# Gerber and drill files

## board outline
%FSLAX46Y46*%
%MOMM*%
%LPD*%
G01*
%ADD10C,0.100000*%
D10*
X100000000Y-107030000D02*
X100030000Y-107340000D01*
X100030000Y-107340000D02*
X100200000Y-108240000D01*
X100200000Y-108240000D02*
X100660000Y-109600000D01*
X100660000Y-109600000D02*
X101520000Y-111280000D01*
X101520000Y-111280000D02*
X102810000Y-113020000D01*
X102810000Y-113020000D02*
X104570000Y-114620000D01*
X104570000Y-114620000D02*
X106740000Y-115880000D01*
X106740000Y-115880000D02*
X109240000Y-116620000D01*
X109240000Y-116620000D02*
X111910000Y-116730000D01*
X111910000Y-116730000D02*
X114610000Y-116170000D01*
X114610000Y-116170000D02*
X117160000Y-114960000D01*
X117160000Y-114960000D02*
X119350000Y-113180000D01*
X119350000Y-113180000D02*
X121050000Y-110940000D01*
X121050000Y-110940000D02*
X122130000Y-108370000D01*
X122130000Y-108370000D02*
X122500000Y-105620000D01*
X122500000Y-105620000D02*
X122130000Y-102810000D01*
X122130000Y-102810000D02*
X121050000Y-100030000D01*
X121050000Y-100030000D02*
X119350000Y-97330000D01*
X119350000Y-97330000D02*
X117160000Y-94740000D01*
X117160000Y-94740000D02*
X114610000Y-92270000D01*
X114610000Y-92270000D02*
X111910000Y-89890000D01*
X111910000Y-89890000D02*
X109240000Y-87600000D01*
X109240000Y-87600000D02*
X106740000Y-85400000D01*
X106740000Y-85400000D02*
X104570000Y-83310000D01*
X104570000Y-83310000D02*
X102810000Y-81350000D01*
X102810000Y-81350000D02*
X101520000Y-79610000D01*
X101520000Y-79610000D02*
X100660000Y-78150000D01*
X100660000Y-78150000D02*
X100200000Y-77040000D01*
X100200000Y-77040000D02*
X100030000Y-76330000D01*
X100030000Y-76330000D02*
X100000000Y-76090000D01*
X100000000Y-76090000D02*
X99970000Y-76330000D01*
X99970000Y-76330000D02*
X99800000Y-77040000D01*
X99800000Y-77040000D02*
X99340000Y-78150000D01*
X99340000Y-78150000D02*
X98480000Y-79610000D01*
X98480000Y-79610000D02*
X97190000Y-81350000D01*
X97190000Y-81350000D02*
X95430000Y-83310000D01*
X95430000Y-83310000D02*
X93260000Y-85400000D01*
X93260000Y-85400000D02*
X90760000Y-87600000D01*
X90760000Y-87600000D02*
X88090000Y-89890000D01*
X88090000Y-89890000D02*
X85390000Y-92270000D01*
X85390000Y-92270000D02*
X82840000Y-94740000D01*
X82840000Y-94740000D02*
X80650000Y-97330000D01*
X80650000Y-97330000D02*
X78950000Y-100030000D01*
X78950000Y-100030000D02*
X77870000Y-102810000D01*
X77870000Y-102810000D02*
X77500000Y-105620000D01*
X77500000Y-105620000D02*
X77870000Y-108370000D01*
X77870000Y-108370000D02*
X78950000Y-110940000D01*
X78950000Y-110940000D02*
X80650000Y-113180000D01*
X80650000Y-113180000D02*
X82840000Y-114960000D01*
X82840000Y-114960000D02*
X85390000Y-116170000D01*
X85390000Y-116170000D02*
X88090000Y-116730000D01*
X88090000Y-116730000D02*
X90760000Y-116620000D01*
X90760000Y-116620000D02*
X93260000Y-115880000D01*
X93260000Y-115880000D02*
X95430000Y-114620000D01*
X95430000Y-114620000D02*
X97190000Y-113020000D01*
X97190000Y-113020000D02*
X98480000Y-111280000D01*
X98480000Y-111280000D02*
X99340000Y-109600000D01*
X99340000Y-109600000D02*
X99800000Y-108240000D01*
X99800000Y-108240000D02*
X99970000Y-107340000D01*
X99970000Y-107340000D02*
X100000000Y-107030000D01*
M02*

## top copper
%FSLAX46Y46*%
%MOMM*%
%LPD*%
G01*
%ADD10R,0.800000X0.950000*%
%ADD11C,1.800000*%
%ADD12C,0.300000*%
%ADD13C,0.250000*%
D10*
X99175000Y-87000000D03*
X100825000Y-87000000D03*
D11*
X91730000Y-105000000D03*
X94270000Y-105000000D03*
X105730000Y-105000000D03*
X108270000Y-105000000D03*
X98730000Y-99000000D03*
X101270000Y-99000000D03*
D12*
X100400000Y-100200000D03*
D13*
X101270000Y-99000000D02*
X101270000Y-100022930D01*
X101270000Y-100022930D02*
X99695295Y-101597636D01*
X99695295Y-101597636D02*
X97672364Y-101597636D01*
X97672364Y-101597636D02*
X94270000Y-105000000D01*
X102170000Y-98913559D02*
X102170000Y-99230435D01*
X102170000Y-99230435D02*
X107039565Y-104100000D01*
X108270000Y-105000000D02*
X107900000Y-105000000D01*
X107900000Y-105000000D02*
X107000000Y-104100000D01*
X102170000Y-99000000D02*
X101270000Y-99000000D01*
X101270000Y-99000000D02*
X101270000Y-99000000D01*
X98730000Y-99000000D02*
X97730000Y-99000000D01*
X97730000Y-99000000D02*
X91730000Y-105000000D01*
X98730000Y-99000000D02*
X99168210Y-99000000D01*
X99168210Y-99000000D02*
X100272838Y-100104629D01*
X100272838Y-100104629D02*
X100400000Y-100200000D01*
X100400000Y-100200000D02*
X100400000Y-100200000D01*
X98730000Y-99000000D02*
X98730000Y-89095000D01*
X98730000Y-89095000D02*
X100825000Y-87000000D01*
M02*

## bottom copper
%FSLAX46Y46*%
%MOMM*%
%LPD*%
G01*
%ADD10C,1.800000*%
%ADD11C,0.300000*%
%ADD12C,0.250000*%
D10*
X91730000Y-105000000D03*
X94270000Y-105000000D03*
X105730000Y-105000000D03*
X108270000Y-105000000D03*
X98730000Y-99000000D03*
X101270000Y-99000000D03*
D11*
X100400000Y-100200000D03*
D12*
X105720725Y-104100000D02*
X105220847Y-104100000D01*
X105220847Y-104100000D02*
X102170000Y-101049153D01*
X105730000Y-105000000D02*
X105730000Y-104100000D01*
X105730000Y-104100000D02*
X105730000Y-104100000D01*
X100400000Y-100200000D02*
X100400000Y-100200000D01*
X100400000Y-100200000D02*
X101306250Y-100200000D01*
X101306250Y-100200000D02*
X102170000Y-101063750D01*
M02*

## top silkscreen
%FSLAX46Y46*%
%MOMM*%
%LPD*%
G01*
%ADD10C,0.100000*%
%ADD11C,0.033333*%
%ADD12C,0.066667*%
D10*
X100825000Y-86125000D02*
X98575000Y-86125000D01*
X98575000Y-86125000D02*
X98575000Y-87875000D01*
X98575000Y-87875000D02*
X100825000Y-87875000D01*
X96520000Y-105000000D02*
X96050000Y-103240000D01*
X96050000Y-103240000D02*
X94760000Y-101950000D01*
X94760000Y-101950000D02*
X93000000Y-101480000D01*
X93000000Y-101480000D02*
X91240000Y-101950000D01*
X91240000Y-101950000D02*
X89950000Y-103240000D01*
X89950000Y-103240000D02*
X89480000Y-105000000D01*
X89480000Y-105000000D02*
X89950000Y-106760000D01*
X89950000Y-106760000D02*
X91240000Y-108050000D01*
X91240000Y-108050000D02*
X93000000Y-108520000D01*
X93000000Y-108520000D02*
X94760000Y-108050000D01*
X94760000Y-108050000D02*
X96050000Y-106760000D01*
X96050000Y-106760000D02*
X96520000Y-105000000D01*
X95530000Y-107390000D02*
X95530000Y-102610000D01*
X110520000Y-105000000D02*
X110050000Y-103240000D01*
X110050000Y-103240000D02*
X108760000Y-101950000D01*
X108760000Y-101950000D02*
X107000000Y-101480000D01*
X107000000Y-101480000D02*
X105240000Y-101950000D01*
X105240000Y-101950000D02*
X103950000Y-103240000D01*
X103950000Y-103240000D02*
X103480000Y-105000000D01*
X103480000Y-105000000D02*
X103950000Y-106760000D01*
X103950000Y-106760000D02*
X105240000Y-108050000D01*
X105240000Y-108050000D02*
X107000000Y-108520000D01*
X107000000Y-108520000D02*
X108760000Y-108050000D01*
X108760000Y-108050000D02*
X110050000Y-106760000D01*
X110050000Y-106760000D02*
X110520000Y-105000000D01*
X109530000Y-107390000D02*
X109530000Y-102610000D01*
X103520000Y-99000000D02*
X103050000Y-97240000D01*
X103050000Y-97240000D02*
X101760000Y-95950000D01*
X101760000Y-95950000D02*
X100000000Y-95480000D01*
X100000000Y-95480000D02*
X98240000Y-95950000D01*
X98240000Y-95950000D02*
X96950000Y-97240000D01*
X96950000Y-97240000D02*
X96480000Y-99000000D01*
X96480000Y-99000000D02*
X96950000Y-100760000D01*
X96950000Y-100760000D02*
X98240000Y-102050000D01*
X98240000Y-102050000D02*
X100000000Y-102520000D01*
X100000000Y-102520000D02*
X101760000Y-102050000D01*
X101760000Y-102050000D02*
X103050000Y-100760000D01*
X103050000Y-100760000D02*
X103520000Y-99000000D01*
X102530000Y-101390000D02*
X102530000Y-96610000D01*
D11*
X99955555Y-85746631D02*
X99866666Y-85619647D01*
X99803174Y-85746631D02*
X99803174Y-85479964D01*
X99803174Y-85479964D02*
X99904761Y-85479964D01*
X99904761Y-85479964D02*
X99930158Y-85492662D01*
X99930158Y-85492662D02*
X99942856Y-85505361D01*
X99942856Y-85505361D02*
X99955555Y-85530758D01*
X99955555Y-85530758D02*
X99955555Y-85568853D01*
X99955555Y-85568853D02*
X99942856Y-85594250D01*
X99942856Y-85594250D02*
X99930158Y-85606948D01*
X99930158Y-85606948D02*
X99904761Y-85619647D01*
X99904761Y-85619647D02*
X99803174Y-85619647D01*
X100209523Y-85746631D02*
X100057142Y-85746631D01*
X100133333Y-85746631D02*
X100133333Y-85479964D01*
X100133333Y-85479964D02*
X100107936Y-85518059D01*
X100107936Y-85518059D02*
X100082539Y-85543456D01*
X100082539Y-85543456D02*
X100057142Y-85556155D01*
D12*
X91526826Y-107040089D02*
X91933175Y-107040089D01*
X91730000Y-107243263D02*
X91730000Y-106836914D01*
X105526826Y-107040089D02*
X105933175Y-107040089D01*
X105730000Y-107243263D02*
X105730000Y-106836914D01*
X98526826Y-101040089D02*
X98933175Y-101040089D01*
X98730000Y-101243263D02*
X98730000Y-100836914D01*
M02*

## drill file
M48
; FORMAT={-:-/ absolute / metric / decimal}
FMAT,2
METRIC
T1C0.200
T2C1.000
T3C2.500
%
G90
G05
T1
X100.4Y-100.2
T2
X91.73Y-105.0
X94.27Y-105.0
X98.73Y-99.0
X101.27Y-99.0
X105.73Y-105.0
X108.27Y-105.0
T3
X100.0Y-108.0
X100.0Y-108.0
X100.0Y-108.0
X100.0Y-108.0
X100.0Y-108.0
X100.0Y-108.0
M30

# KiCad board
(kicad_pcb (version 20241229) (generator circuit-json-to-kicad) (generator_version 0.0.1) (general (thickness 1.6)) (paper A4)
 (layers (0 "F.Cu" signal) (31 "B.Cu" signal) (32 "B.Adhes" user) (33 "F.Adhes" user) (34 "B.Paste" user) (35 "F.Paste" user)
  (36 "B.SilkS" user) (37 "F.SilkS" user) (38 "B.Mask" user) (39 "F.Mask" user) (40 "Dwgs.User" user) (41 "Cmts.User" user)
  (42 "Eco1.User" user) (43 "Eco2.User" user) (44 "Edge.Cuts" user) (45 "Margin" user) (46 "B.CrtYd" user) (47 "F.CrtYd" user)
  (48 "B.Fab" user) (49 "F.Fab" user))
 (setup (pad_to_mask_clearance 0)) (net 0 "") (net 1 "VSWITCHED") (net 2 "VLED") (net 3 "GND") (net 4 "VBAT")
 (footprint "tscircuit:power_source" (layer F.Cu) (at 100 95 0)
  (pad "" np_thru_hole circle (at 0 13 0) (size 2.5 2.5) (drill 2.5) (layers *.Cu *.Mask)))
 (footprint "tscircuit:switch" (layer F.Cu) (at 100 90 0)
  (pad "" np_thru_hole circle (at 0 18 0) (size 2.5 2.5) (drill 2.5) (layers *.Cu *.Mask)))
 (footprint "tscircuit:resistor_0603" (layer F.Cu) (at 100 87 0)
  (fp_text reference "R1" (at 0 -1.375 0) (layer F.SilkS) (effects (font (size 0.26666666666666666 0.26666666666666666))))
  (pad "1" smd rect (at -0.825 0 0) (size 0.8 0.95) (layers F.Cu F.Paste F.Mask) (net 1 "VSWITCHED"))
  (pad "2" smd rect (at 0.825 0 0) (size 0.8 0.95) (layers F.Cu F.Paste F.Mask) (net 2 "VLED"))
  (pad "" np_thru_hole circle (at 0 21 0) (size 2.5 2.5) (drill 2.5) (layers *.Cu *.Mask)))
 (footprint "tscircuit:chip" (layer F.Cu) (at 93 105 0)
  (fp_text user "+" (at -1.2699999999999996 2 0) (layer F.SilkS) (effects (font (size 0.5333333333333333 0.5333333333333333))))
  (pad "1" thru_hole circle (at -1.2699999999999996 0 0) (size 1.8 1.8) (drill 1) (layers *.Cu *.Mask) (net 2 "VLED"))
  (pad "2" thru_hole circle (at 1.2699999999999996 0 0) (size 1.8 1.8) (drill 1) (layers *.Cu *.Mask) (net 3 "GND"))
  (pad "" np_thru_hole circle (at 7 3 0) (size 2.5 2.5) (drill 2.5) (layers *.Cu *.Mask)))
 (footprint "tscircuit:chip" (layer F.Cu) (at 107 105 0)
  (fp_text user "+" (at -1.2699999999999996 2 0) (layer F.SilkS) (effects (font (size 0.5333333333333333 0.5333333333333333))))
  (pad "1" thru_hole circle (at -1.2699999999999996 0 0) (size 1.8 1.8) (drill 1) (layers *.Cu *.Mask) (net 2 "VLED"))
  (pad "2" thru_hole circle (at 1.2699999999999996 0 0) (size 1.8 1.8) (drill 1) (layers *.Cu *.Mask) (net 3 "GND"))
  (pad "" np_thru_hole circle (at -7 3 0) (size 2.5 2.5) (drill 2.5) (layers *.Cu *.Mask)))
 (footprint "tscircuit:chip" (layer F.Cu) (at 100 99 0)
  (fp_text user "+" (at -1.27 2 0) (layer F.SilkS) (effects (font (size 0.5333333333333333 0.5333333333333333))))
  (pad "1" thru_hole circle (at -1.27 0 0) (size 1.8 1.8) (drill 1) (layers *.Cu *.Mask) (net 2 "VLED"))
  (pad "2" thru_hole circle (at 1.27 0 0) (size 1.8 1.8) (drill 1) (layers *.Cu *.Mask) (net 3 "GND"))
  (pad "" np_thru_hole circle (at 0 9 0) (size 2.5 2.5) (drill 2.5) (layers *.Cu *.Mask)))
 (segment (start 101.27 99) (end 101.27 100.02293031919105) (width 0.25) (layer F.Cu) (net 3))
 (segment (start 101.27 100.02293031919105) (end 99.69529453119956 101.59763578799148) (width 0.25) (layer F.Cu) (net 3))
 (segment (start 99.69529453119956 101.59763578799148) (end 97.67236421200852 101.59763578799148) (width 0.25) (layer F.Cu) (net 3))
 (segment (start 97.67236421200852 101.59763578799148) (end 94.27 105) (width 0.25) (layer F.Cu) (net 3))
 (segment (start 102.17 98.9135593220339) (end 102.17 99.2304347826087) (width 0.25) (layer F.Cu) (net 3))
 (segment (start 102.17 99.2304347826087) (end 107.0395652173913 104.1) (width 0.25) (layer F.Cu) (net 3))
 (segment (start 108.27 105) (end 107.9 105) (width 0.25) (layer F.Cu) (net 3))
 (segment (start 107.9 105) (end 107 104.1) (width 0.25) (layer F.Cu) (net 3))
 (segment (start 102.17 99) (end 101.27 99) (width 0.25) (layer F.Cu) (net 3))
 (segment (start 101.27 99) (end 101.27 99) (width 0.25) (layer F.Cu) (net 3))
 (segment (start 98.73 99) (end 97.73 99) (width 0.25) (layer F.Cu) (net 2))
 (segment (start 97.73 99) (end 91.73 105) (width 0.25) (layer F.Cu) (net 2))
 (segment (start 105.72072463768116 104.1) (end 105.22084745762712 104.1) (width 0.25) (layer B.Cu) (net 2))
 (segment (start 105.22084745762712 104.1) (end 102.17 101.04915254237288) (width 0.25) (layer B.Cu) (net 2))
 (segment (start 105.73 105) (end 105.73 104.1) (width 0.25) (layer B.Cu) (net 2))
 (segment (start 105.73 104.1) (end 105.73 104.1) (width 0.25) (layer B.Cu) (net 2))
 (segment (start 98.73 99) (end 99.1682096086742 99) (width 0.25) (layer F.Cu) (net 2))
 (segment (start 99.1682096086742 99) (end 100.27283843469682 100.10462882602262) (width 0.25) (layer F.Cu) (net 2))
 (segment (start 100.27283843469682 100.10462882602262) (end 100.4 100.2) (width 0.25) (layer F.Cu) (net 2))
 (segment (start 100.4 100.2) (end 100.4 100.2) (width 0.25) (layer F.Cu) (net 2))
 (segment (start 100.4 100.2) (end 100.4 100.2) (width 0.25) (layer B.Cu) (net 2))
 (segment (start 100.4 100.2) (end 101.30625 100.2) (width 0.25) (layer B.Cu) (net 2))
 (segment (start 101.30625 100.2) (end 102.17 101.06375) (width 0.25) (layer B.Cu) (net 2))
 (segment (start 98.73 99) (end 98.73 89.095) (width 0.25) (layer F.Cu) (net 2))
 (segment (start 98.73 89.095) (end 100.825 87) (width 0.25) (layer F.Cu) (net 2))
 (gr_line (start 100.825 86.125) (end 98.575 86.125) (width 0.1) (layer F.SilkS))
 (gr_line (start 98.575 86.125) (end 98.575 87.875) (width 0.1) (layer F.SilkS))
 (gr_line (start 98.575 87.875) (end 100.825 87.875) (width 0.1) (layer F.SilkS))
 (gr_line (start 96.52 105) (end 96.05 103.24) (width 0.1) (layer F.SilkS))
 (gr_line (start 96.05 103.24) (end 94.76 101.95) (width 0.1) (layer F.SilkS))
 (gr_line (start 94.76 101.95) (end 93 101.48) (width 0.1) (layer F.SilkS))
 (gr_line (start 93 101.48) (end 91.24 101.95) (width 0.1) (layer F.SilkS))
 (gr_line (start 91.24 101.95) (end 89.95 103.24) (width 0.1) (layer F.SilkS))
 (gr_line (start 89.95 103.24) (end 89.48 105) (width 0.1) (layer F.SilkS))
 (gr_line (start 89.48 105) (end 89.95 106.76) (width 0.1) (layer F.SilkS))
 (gr_line (start 89.95 106.76) (end 91.24 108.05) (width 0.1) (layer F.SilkS))
 (gr_line (start 91.24 108.05) (end 93 108.52) (width 0.1) (layer F.SilkS))
 (gr_line (start 93 108.52) (end 94.76 108.05) (width 0.1) (layer F.SilkS))
 (gr_line (start 94.76 108.05) (end 96.05 106.76) (width 0.1) (layer F.SilkS))
 (gr_line (start 96.05 106.76) (end 96.52 105) (width 0.1) (layer F.SilkS))
 (gr_line (start 95.53 107.39) (end 95.53 102.61) (width 0.1) (layer F.SilkS))
 (gr_line (start 110.52 105) (end 110.05 103.24) (width 0.1) (layer F.SilkS))
 (gr_line (start 110.05 103.24) (end 108.76 101.95) (width 0.1) (layer F.SilkS))
 (gr_line (start 108.76 101.95) (end 107 101.48) (width 0.1) (layer F.SilkS))
 (gr_line (start 107 101.48) (end 105.24 101.95) (width 0.1) (layer F.SilkS))
 (gr_line (start 105.24 101.95) (end 103.95 103.24) (width 0.1) (layer F.SilkS))
 (gr_line (start 103.95 103.24) (end 103.48 105) (width 0.1) (layer F.SilkS))
 (gr_line (start 103.48 105) (end 103.95 106.76) (width 0.1) (layer F.SilkS))
 (gr_line (start 103.95 106.76) (end 105.24 108.05) (width 0.1) (layer F.SilkS))
 (gr_line (start 105.24 108.05) (end 107 108.52) (width 0.1) (layer F.SilkS))
 (gr_line (start 107 108.52) (end 108.76 108.05) (width 0.1) (layer F.SilkS))
 (gr_line (start 108.76 108.05) (end 110.05 106.76) (width 0.1) (layer F.SilkS))
 (gr_line (start 110.05 106.76) (end 110.52 105) (width 0.1) (layer F.SilkS))
 (gr_line (start 109.53 107.39) (end 109.53 102.61) (width 0.1) (layer F.SilkS))
 (gr_line (start 103.52 99) (end 103.05 97.24) (width 0.1) (layer F.SilkS))
 (gr_line (start 103.05 97.24) (end 101.76 95.95) (width 0.1) (layer F.SilkS))
 (gr_line (start 101.76 95.95) (end 100 95.48) (width 0.1) (layer F.SilkS))
 (gr_line (start 100 95.48) (end 98.24 95.95) (width 0.1) (layer F.SilkS))
 (gr_line (start 98.24 95.95) (end 96.95 97.24) (width 0.1) (layer F.SilkS))
 (gr_line (start 96.95 97.24) (end 96.48 99) (width 0.1) (layer F.SilkS))
 (gr_line (start 96.48 99) (end 96.95 100.76) (width 0.1) (layer F.SilkS))
 (gr_line (start 96.95 100.76) (end 98.24 102.05) (width 0.1) (layer F.SilkS))
 (gr_line (start 98.24 102.05) (end 100 102.52) (width 0.1) (layer F.SilkS))
 (gr_line (start 100 102.52) (end 101.76 102.05) (width 0.1) (layer F.SilkS))
 (gr_line (start 101.76 102.05) (end 103.05 100.76) (width 0.1) (layer F.SilkS))
 (gr_line (start 103.05 100.76) (end 103.52 99) (width 0.1) (layer F.SilkS))
 (gr_line (start 102.53 101.39) (end 102.53 96.61) (width 0.1) (layer F.SilkS))
 (gr_line (start 100 107.03) (end 100.03 107.34) (width 0.1) (layer Edge.Cuts))
 (gr_line (start 100.03 107.34) (end 100.2 108.24) (width 0.1) (layer Edge.Cuts))
 (gr_line (start 100.2 108.24) (end 100.66 109.6) (width 0.1) (layer Edge.Cuts))
 (gr_line (start 100.66 109.6) (end 101.52 111.28) (width 0.1) (layer Edge.Cuts))
 (gr_line (start 101.52 111.28) (end 102.81 113.02) (width 0.1) (layer Edge.Cuts))
 (gr_line (start 102.81 113.02) (end 104.57 114.62) (width 0.1) (layer Edge.Cuts))
 (gr_line (start 104.57 114.62) (end 106.74 115.88) (width 0.1) (layer Edge.Cuts))
 (gr_line (start 106.74 115.88) (end 109.24 116.62) (width 0.1) (layer Edge.Cuts))
 (gr_line (start 109.24 116.62) (end 111.91 116.73) (width 0.1) (layer Edge.Cuts))
 (gr_line (start 111.91 116.73) (end 114.61 116.17) (width 0.1) (layer Edge.Cuts))
 (gr_line (start 114.61 116.17) (end 117.16 114.96000000000001) (width 0.1) (layer Edge.Cuts))
 (gr_line (start 117.16 114.96000000000001) (end 119.35 113.18) (width 0.1) (layer Edge.Cuts))
 (gr_line (start 119.35 113.18) (end 121.05 110.94) (width 0.1) (layer Edge.Cuts))
 (gr_line (start 121.05 110.94) (end 122.13 108.37) (width 0.1) (layer Edge.Cuts))
 (gr_line (start 122.13 108.37) (end 122.5 105.62) (width 0.1) (layer Edge.Cuts))
 (gr_line (start 122.5 105.62) (end 122.13 102.81) (width 0.1) (layer Edge.Cuts))
 (gr_line (start 122.13 102.81) (end 121.05 100.03) (width 0.1) (layer Edge.Cuts))
 (gr_line (start 121.05 100.03) (end 119.35 97.33) (width 0.1) (layer Edge.Cuts))
 (gr_line (start 119.35 97.33) (end 117.16 94.74) (width 0.1) (layer Edge.Cuts))
 (gr_line (start 117.16 94.74) (end 114.61 92.27) (width 0.1) (layer Edge.Cuts))
 (gr_line (start 114.61 92.27) (end 111.91 89.89) (width 0.1) (layer Edge.Cuts))
 (gr_line (start 111.91 89.89) (end 109.24 87.6) (width 0.1) (layer Edge.Cuts))
 (gr_line (start 109.24 87.6) (end 106.74 85.4) (width 0.1) (layer Edge.Cuts))
 (gr_line (start 106.74 85.4) (end 104.57 83.31) (width 0.1) (layer Edge.Cuts))
 (gr_line (start 104.57 83.31) (end 102.81 81.35) (width 0.1) (layer Edge.Cuts))
 (gr_line (start 102.81 81.35) (end 101.52 79.61) (width 0.1) (layer Edge.Cuts))
 (gr_line (start 101.52 79.61) (end 100.66 78.15) (width 0.1) (layer Edge.Cuts))
 (gr_line (start 100.66 78.15) (end 100.2 77.03999999999999) (width 0.1) (layer Edge.Cuts))
 (gr_line (start 100.2 77.03999999999999) (end 100.03 76.33) (width 0.1) (layer Edge.Cuts))
 (gr_line (start 100.03 76.33) (end 100 76.09) (width 0.1) (layer Edge.Cuts))
 (gr_line (start 100 76.09) (end 99.97 76.33) (width 0.1) (layer Edge.Cuts))
 (gr_line (start 99.97 76.33) (end 99.8 77.03999999999999) (width 0.1) (layer Edge.Cuts))
 (gr_line (start 99.8 77.03999999999999) (end 99.34 78.15) (width 0.1) (layer Edge.Cuts))
 (gr_line (start 99.34 78.15) (end 98.48 79.61) (width 0.1) (layer Edge.Cuts))
 (gr_line (start 98.48 79.61) (end 97.19 81.35) (width 0.1) (layer Edge.Cuts))
 (gr_line (start 97.19 81.35) (end 95.43 83.31) (width 0.1) (layer Edge.Cuts))
 (gr_line (start 95.43 83.31) (end 93.26 85.4) (width 0.1) (layer Edge.Cuts))
 (gr_line (start 93.26 85.4) (end 90.76 87.6) (width 0.1) (layer Edge.Cuts))
 (gr_line (start 90.76 87.6) (end 88.09 89.89) (width 0.1) (layer Edge.Cuts))
 (gr_line (start 88.09 89.89) (end 85.39 92.27) (width 0.1) (layer Edge.Cuts))
 (gr_line (start 85.39 92.27) (end 82.84 94.74) (width 0.1) (layer Edge.Cuts))
 (gr_line (start 82.84 94.74) (end 80.65 97.33) (width 0.1) (layer Edge.Cuts))
 (gr_line (start 80.65 97.33) (end 78.95 100.03) (width 0.1) (layer Edge.Cuts))
 (gr_line (start 78.95 100.03) (end 77.87 102.81) (width 0.1) (layer Edge.Cuts))
 (gr_line (start 77.87 102.81) (end 77.5 105.62) (width 0.1) (layer Edge.Cuts))
 (gr_line (start 77.5 105.62) (end 77.87 108.37) (width 0.1) (layer Edge.Cuts))
 (gr_line (start 77.87 108.37) (end 78.95 110.94) (width 0.1) (layer Edge.Cuts))
 (gr_line (start 78.95 110.94) (end 80.65 113.18) (width 0.1) (layer Edge.Cuts))
 (gr_line (start 80.65 113.18) (end 82.84 114.96000000000001) (width 0.1) (layer Edge.Cuts))
 (gr_line (start 82.84 114.96000000000001) (end 85.39 116.17) (width 0.1) (layer Edge.Cuts))
 (gr_line (start 85.39 116.17) (end 88.09 116.73) (width 0.1) (layer Edge.Cuts))
 (gr_line (start 88.09 116.73) (end 90.76 116.62) (width 0.1) (layer Edge.Cuts))
 (gr_line (start 90.76 116.62) (end 93.26 115.88) (width 0.1) (layer Edge.Cuts))
 (gr_line (start 93.26 115.88) (end 95.43 114.62) (width 0.1) (layer Edge.Cuts))
 (gr_line (start 95.43 114.62) (end 97.19 113.02) (width 0.1) (layer Edge.Cuts))
 (gr_line (start 97.19 113.02) (end 98.48 111.28) (width 0.1) (layer Edge.Cuts))
 (gr_line (start 98.48 111.28) (end 99.34 109.6) (width 0.1) (layer Edge.Cuts))
 (gr_line (start 99.34 109.6) (end 99.8 108.24) (width 0.1) (layer Edge.Cuts))
 (gr_line (start 99.8 108.24) (end 99.97 107.34) (width 0.1) (layer Edge.Cuts))
 (gr_line (start 99.97 107.34) (end 100 107.03) (width 0.1) (layer Edge.Cuts))
 (via (at 100.4 100.2) (size 0.3) (drill 0.2) (layers F.Cu B.Cu) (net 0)))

